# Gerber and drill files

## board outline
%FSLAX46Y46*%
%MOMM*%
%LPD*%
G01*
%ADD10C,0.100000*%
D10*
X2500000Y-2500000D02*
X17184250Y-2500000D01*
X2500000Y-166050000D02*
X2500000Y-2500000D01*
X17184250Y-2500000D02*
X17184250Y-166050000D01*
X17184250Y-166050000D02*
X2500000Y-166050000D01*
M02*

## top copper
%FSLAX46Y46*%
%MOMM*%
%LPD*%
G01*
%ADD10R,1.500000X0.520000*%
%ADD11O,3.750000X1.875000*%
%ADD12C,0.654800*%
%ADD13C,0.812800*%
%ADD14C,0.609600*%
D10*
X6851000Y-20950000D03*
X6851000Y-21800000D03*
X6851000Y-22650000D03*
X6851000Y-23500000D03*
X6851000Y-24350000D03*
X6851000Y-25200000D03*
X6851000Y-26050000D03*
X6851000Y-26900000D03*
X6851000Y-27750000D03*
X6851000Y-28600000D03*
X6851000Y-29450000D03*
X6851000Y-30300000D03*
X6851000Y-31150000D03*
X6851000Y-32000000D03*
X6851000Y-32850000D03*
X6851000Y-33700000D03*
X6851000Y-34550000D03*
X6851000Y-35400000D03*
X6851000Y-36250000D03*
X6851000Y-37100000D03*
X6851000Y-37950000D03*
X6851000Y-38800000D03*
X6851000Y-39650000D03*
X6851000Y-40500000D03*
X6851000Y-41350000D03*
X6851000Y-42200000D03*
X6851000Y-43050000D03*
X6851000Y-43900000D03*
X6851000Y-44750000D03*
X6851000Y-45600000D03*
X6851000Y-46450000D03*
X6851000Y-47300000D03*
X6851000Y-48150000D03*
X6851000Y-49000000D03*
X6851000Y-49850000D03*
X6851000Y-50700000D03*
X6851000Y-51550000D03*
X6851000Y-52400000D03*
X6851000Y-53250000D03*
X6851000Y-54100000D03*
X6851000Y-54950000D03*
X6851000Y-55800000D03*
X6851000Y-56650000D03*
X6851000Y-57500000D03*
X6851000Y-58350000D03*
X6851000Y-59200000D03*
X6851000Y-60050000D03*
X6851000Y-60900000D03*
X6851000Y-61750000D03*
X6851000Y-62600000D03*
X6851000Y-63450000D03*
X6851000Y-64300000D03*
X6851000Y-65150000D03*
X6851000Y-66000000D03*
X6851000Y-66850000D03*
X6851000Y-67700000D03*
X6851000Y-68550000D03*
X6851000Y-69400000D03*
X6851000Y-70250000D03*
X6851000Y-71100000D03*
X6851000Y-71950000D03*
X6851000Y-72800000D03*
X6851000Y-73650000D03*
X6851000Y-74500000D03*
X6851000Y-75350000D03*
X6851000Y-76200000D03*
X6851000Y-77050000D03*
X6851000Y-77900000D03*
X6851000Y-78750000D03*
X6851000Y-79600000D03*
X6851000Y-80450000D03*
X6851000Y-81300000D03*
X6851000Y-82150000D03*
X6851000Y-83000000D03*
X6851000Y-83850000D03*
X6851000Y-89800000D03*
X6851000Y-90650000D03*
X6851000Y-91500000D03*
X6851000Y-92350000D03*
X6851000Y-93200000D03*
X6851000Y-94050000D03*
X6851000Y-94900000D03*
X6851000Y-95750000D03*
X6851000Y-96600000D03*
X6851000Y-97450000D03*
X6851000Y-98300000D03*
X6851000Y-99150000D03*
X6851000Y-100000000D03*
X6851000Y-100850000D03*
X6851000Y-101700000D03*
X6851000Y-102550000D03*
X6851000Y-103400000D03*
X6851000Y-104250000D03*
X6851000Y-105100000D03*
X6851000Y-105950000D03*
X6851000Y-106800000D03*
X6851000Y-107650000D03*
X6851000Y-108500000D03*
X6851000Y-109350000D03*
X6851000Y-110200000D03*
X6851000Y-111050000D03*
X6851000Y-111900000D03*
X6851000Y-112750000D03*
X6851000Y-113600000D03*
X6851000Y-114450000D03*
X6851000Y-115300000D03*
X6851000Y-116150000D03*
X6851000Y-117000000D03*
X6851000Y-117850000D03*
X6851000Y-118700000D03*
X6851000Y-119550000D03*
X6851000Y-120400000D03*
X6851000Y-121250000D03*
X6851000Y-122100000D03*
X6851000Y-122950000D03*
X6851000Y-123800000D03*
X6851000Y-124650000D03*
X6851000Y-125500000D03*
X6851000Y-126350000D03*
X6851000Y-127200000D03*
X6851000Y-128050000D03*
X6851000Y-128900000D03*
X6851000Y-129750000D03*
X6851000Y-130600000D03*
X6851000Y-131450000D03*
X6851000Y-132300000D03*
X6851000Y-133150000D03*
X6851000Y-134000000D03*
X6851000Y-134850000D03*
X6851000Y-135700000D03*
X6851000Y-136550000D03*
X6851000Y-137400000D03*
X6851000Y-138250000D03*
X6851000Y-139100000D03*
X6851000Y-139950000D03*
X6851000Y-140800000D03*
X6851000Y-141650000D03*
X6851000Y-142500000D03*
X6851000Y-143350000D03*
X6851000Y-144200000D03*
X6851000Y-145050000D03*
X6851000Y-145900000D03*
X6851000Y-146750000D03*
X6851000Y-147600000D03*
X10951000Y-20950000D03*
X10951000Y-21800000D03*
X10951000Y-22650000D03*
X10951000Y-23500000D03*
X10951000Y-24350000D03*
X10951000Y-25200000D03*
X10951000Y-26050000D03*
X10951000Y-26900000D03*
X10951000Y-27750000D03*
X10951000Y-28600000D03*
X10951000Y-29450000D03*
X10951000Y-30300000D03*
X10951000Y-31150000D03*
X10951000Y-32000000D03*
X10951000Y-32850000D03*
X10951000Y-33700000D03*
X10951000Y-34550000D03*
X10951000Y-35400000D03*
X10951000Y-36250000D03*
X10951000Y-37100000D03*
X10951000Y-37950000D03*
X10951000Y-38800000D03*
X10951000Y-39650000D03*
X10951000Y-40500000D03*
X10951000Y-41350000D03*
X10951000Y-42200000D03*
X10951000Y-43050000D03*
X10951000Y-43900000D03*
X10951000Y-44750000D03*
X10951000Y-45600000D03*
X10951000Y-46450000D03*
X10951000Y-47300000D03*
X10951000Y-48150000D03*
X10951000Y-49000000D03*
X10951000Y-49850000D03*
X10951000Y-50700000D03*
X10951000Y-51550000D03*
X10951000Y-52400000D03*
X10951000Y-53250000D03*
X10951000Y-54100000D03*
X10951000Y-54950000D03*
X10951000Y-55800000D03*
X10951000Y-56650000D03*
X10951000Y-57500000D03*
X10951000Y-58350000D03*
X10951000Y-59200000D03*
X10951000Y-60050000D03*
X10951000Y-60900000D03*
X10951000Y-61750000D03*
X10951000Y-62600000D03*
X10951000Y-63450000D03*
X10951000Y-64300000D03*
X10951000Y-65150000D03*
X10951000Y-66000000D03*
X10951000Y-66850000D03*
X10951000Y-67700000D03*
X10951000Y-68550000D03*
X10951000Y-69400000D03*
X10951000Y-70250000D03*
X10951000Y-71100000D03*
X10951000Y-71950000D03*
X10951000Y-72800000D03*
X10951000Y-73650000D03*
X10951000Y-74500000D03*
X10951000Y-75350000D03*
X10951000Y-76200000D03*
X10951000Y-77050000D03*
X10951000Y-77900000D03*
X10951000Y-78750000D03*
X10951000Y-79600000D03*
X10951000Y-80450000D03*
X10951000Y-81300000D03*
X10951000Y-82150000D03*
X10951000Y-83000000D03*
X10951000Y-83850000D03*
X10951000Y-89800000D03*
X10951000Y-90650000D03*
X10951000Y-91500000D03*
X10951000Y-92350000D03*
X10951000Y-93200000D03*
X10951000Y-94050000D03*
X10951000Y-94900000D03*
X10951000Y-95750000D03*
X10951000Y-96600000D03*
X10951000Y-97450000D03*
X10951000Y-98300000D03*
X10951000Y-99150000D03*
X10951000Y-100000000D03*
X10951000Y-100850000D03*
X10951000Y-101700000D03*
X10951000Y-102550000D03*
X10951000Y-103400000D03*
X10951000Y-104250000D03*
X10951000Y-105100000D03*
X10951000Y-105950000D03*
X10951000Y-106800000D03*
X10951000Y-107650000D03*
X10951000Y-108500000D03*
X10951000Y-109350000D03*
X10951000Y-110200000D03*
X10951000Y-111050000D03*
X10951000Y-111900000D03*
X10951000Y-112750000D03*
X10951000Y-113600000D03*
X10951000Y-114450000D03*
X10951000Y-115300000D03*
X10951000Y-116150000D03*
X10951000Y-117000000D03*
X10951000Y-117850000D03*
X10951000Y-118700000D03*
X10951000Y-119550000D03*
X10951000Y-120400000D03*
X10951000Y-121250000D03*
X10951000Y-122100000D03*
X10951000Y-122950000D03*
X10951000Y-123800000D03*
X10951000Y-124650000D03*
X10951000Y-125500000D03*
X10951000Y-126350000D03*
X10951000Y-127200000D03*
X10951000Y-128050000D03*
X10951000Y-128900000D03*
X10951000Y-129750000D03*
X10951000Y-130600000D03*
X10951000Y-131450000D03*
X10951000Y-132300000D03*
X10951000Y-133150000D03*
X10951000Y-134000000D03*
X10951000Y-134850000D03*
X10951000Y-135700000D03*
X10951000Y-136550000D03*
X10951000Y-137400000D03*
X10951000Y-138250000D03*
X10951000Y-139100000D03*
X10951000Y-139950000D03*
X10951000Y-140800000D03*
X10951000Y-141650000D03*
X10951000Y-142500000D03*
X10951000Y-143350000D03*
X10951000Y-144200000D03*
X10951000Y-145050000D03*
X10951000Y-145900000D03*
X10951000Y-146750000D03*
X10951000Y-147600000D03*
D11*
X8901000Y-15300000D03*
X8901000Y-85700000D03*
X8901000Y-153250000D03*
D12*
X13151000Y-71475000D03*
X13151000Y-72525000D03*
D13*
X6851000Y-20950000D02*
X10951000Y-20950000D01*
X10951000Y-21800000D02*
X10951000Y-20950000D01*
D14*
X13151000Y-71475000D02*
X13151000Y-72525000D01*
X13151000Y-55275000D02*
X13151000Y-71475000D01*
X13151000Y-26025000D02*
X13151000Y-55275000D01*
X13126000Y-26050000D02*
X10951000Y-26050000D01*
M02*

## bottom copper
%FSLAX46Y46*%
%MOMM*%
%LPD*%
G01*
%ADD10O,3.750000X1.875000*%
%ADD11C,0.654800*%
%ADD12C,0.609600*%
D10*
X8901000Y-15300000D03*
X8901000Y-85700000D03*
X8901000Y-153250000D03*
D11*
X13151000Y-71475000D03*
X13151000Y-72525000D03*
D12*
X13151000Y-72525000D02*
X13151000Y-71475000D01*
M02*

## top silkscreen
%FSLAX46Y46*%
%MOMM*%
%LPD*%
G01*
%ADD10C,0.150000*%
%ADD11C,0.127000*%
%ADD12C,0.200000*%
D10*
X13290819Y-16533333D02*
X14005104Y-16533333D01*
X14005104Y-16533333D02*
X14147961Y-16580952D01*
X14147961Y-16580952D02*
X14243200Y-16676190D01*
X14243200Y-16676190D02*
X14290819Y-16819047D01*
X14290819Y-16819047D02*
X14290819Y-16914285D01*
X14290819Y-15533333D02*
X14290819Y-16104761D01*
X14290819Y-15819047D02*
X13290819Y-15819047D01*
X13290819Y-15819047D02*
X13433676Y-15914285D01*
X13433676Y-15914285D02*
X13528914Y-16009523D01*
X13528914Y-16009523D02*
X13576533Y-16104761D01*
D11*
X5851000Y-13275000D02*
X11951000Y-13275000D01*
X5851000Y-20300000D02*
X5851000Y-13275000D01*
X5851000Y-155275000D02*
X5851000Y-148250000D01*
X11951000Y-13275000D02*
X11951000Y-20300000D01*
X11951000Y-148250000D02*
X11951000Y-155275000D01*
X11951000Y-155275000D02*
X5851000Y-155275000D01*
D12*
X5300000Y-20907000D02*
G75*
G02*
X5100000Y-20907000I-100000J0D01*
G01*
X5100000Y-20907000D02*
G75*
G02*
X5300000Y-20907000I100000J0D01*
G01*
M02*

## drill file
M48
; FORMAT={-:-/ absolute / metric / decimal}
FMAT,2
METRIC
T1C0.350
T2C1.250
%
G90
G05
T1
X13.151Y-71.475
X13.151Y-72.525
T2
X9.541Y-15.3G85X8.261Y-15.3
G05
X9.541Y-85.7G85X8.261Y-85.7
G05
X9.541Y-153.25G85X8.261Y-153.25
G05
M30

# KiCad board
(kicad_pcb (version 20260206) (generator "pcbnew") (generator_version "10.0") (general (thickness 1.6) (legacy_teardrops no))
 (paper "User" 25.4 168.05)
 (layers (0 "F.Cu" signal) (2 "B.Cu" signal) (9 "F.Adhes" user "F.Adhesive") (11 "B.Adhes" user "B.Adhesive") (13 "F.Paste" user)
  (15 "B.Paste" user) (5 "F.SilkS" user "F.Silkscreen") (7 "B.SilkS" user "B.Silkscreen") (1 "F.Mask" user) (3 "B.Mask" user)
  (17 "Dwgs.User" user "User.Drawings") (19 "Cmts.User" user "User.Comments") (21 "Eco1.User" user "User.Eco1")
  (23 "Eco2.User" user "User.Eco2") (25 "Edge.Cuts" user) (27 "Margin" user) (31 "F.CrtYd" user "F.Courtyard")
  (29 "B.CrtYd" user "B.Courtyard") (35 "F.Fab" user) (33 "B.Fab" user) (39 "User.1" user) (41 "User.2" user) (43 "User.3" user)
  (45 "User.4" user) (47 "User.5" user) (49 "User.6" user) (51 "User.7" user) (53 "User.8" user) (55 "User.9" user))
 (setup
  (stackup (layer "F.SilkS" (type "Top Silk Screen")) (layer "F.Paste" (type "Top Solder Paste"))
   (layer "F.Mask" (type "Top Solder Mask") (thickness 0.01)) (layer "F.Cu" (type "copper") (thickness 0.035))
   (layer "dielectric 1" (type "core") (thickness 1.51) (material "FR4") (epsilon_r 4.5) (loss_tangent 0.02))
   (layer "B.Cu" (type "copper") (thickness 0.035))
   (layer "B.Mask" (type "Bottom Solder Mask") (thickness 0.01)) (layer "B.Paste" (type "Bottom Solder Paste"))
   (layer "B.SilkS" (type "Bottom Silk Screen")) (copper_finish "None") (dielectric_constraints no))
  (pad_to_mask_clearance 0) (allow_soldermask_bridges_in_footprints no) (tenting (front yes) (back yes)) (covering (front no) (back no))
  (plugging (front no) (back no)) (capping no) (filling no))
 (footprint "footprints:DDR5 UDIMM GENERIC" (layer "F.Cu") (at 8.901 84.275 -90)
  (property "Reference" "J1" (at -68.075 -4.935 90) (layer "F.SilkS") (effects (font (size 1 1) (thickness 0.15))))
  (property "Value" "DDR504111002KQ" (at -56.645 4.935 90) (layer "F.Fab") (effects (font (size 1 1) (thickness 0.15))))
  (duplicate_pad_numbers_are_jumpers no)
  (fp_line (start -71 3.05) (end -71 -3.05) (stroke (width 0.127) (type solid)) (layer "F.SilkS"))
  (fp_line (start -63.975 3.05) (end -71 3.05) (stroke (width 0.127) (type solid)) (layer "F.SilkS"))
  (fp_line (start 71 3.05) (end 63.975 3.05) (stroke (width 0.127) (type solid)) (layer "F.SilkS"))
  (fp_line (start -71 -3.05) (end -63.975 -3.05) (stroke (width 0.127) (type solid)) (layer "F.SilkS"))
  (fp_line (start 63.975 -3.05) (end 71 -3.05) (stroke (width 0.127) (type solid)) (layer "F.SilkS"))
  (fp_line (start 71 -3.05) (end 71 3.05) (stroke (width 0.127) (type solid)) (layer "F.SilkS"))
  (fp_circle (center -63.368 3.701) (end -63.268 3.701) (stroke (width 0.2) (type solid)) (fill no) (layer "F.SilkS"))
  (pad "01" smd rect (at -63.325 2.05 270) (size 0.52 1.5) (layers "F.Cu" "F.Mask" "F.Paste") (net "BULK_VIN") (solder_mask_margin 0.102))
  (pad "02" smd rect (at -62.475 2.05 270) (size 0.52 1.5) (layers "F.Cu" "F.Mask" "F.Paste") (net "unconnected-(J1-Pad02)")
   (solder_mask_margin 0.102))
  (pad "03" smd rect (at -61.625 2.05 270) (size 0.52 1.5) (layers "F.Cu" "F.Mask" "F.Paste") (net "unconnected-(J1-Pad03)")
   (solder_mask_margin 0.102))
  (pad "04" smd rect (at -60.775 2.05 270) (size 0.52 1.5) (layers "F.Cu" "F.Mask" "F.Paste") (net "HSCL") (solder_mask_margin 0.102))
  (pad "05" smd rect (at -59.925 2.05 270) (size 0.52 1.5) (layers "F.Cu" "F.Mask" "F.Paste") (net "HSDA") (solder_mask_margin 0.102))
  (pad "06" smd rect (at -59.075 2.05 270) (size 0.52 1.5) (layers "F.Cu" "F.Mask" "F.Paste") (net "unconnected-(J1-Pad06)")
   (solder_mask_margin 0.102))
  (pad "07" smd rect (at -58.225 2.05 270) (size 0.52 1.5) (layers "F.Cu" "F.Mask" "F.Paste") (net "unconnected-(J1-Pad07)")
   (solder_mask_margin 0.102))
  (pad "08" smd rect (at -57.375 2.05 270) (size 0.52 1.5) (layers "F.Cu" "F.Mask" "F.Paste") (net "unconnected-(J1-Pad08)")
   (solder_mask_margin 0.102))
  (pad "09" smd rect (at -56.525 2.05 270) (size 0.52 1.5) (layers "F.Cu" "F.Mask" "F.Paste") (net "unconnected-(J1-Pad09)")
   (solder_mask_margin 0.102))
  (pad "10" smd rect (at -55.675 2.05 270) (size 0.52 1.5) (layers "F.Cu" "F.Mask" "F.Paste") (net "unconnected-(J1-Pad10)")
   (solder_mask_margin 0.102))
  (pad "11" smd rect (at -54.825 2.05 270) (size 0.52 1.5) (layers "F.Cu" "F.Mask" "F.Paste") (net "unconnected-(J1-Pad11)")
   (solder_mask_margin 0.102))
  (pad "12" smd rect (at -53.975 2.05 270) (size 0.52 1.5) (layers "F.Cu" "F.Mask" "F.Paste") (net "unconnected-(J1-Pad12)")
   (solder_mask_margin 0.102))
  (pad "13" smd rect (at -53.125 2.05 270) (size 0.52 1.5) (layers "F.Cu" "F.Mask" "F.Paste") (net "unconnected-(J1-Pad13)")
   (solder_mask_margin 0.102))
  (pad "14" smd rect (at -52.275 2.05 270) (size 0.52 1.5) (layers "F.Cu" "F.Mask" "F.Paste") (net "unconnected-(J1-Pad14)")
   (solder_mask_margin 0.102))
  (pad "15" smd rect (at -51.425 2.05 270) (size 0.52 1.5) (layers "F.Cu" "F.Mask" "F.Paste") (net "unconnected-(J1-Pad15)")
   (solder_mask_margin 0.102))
  (pad "16" smd rect (at -50.575 2.05 270) (size 0.52 1.5) (layers "F.Cu" "F.Mask" "F.Paste") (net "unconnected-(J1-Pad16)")
   (solder_mask_margin 0.102))
  (pad "17" smd rect (at -49.725 2.05 270) (size 0.52 1.5) (layers "F.Cu" "F.Mask" "F.Paste") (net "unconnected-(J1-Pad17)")
   (solder_mask_margin 0.102))
  (pad "18" smd rect (at -48.875 2.05 270) (size 0.52 1.5) (layers "F.Cu" "F.Mask" "F.Paste") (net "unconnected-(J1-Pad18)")
   (solder_mask_margin 0.102))
  (pad "19" smd rect (at -48.025 2.05 270) (size 0.52 1.5) (layers "F.Cu" "F.Mask" "F.Paste") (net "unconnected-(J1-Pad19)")
   (solder_mask_margin 0.102))
  (pad "20" smd rect (at -47.175 2.05 270) (size 0.52 1.5) (layers "F.Cu" "F.Mask" "F.Paste") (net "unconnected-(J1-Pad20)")
   (solder_mask_margin 0.102))
  (pad "21" smd rect (at -46.325 2.05 270) (size 0.52 1.5) (layers "F.Cu" "F.Mask" "F.Paste") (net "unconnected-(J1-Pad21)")
   (solder_mask_margin 0.102))
  (pad "22" smd rect (at -45.475 2.05 270) (size 0.52 1.5) (layers "F.Cu" "F.Mask" "F.Paste") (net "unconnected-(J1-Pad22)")
   (solder_mask_margin 0.102))
  (pad "23" smd rect (at -44.625 2.05 270) (size 0.52 1.5) (layers "F.Cu" "F.Mask" "F.Paste") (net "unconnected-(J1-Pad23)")
   (solder_mask_margin 0.102))
  (pad "24" smd rect (at -43.775 2.05 270) (size 0.52 1.5) (layers "F.Cu" "F.Mask" "F.Paste") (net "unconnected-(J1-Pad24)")
   (solder_mask_margin 0.102))
  (pad "25" smd rect (at -42.925 2.05 270) (size 0.52 1.5) (layers "F.Cu" "F.Mask" "F.Paste") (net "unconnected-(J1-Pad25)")
   (solder_mask_margin 0.102))
  (pad "26" smd rect (at -42.075 2.05 270) (size 0.52 1.5) (layers "F.Cu" "F.Mask" "F.Paste") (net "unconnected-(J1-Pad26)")
   (solder_mask_margin 0.102))
  (pad "27" smd rect (at -41.225 2.05 270) (size 0.52 1.5) (layers "F.Cu" "F.Mask" "F.Paste") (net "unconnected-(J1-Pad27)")
   (solder_mask_margin 0.102))
  (pad "28" smd rect (at -40.375 2.05 270) (size 0.52 1.5) (layers "F.Cu" "F.Mask" "F.Paste") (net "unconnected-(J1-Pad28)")
   (solder_mask_margin 0.102))
  (pad "29" smd rect (at -39.525 2.05 270) (size 0.52 1.5) (layers "F.Cu" "F.Mask" "F.Paste") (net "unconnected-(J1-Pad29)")
   (solder_mask_margin 0.102))
  (pad "30" smd rect (at -38.675 2.05 270) (size 0.52 1.5) (layers "F.Cu" "F.Mask" "F.Paste") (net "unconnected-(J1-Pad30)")
   (solder_mask_margin 0.102))
  (pad "31" smd rect (at -37.825 2.05 270) (size 0.52 1.5) (layers "F.Cu" "F.Mask" "F.Paste") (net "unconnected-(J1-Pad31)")
   (solder_mask_margin 0.102))
  (pad "32" smd rect (at -36.975 2.05 270) (size 0.52 1.5) (layers "F.Cu" "F.Mask" "F.Paste") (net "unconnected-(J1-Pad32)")
   (solder_mask_margin 0.102))
  (pad "33" smd rect (at -36.125 2.05 270) (size 0.52 1.5) (layers "F.Cu" "F.Mask" "F.Paste") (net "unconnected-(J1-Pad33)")
   (solder_mask_margin 0.102))
  (pad "34" smd rect (at -35.275 2.05 270) (size 0.52 1.5) (layers "F.Cu" "F.Mask" "F.Paste") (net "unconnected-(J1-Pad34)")
   (solder_mask_margin 0.102))
  (pad "35" smd rect (at -34.425 2.05 270) (size 0.52 1.5) (layers "F.Cu" "F.Mask" "F.Paste") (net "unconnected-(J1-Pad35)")
   (solder_mask_margin 0.102))
  (pad "36" smd rect (at -33.575 2.05 270) (size 0.52 1.5) (layers "F.Cu" "F.Mask" "F.Paste") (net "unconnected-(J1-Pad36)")
   (solder_mask_margin 0.102))
  (pad "37" smd rect (at -32.725 2.05 270) (size 0.52 1.5) (layers "F.Cu" "F.Mask" "F.Paste") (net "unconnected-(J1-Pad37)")
   (solder_mask_margin 0.102))
  (pad "38" smd rect (at -31.875 2.05 270) (size 0.52 1.5) (layers "F.Cu" "F.Mask" "F.Paste") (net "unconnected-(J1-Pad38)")
   (solder_mask_margin 0.102))
  (pad "39" smd rect (at -31.025 2.05 270) (size 0.52 1.5) (layers "F.Cu" "F.Mask" "F.Paste") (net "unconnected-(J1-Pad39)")
   (solder_mask_margin 0.102))
  (pad "40" smd rect (at -30.175 2.05 270) (size 0.52 1.5) (layers "F.Cu" "F.Mask" "F.Paste") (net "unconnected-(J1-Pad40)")
   (solder_mask_margin 0.102))
  (pad "41" smd rect (at -29.325 2.05 270) (size 0.52 1.5) (layers "F.Cu" "F.Mask" "F.Paste") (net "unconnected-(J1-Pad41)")
   (solder_mask_margin 0.102))
  (pad "42" smd rect (at -28.475 2.05 270) (size 0.52 1.5) (layers "F.Cu" "F.Mask" "F.Paste") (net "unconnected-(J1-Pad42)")
   (solder_mask_margin 0.102))
  (pad "43" smd rect (at -27.625 2.05 270) (size 0.52 1.5) (layers "F.Cu" "F.Mask" "F.Paste") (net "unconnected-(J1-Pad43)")
   (solder_mask_margin 0.102))
  (pad "44" smd rect (at -26.775 2.05 270) (size 0.52 1.5) (layers "F.Cu" "F.Mask" "F.Paste") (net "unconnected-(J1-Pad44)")
   (solder_mask_margin 0.102))
  (pad "45" smd rect (at -25.925 2.05 270) (size 0.52 1.5) (layers "F.Cu" "F.Mask" "F.Paste") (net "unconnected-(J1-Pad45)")
   (solder_mask_margin 0.102))
  (pad "46" smd rect (at -25.075 2.05 270) (size 0.52 1.5) (layers "F.Cu" "F.Mask" "F.Paste") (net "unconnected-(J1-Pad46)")
   (solder_mask_margin 0.102))
  (pad "47" smd rect (at -24.225 2.05 270) (size 0.52 1.5) (layers "F.Cu" "F.Mask" "F.Paste") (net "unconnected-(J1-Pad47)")
   (solder_mask_margin 0.102))
  (pad "48" smd rect (at -23.375 2.05 270) (size 0.52 1.5) (layers "F.Cu" "F.Mask" "F.Paste") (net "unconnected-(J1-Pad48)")
   (solder_mask_margin 0.102))
  (pad "49" smd rect (at -22.525 2.05 270) (size 0.52 1.5) (layers "F.Cu" "F.Mask" "F.Paste") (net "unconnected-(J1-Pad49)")
   (solder_mask_margin 0.102))
  (pad "50" smd rect (at -21.675 2.05 270) (size 0.52 1.5) (layers "F.Cu" "F.Mask" "F.Paste") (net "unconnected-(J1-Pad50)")
   (solder_mask_margin 0.102))
  (pad "51" smd rect (at -20.825 2.05 270) (size 0.52 1.5) (layers "F.Cu" "F.Mask" "F.Paste") (solder_mask_margin 0.102))
  (pad "52" smd rect (at -19.975 2.05 270) (size 0.52 1.5) (layers "F.Cu" "F.Mask" "F.Paste") (solder_mask_margin 0.102))
  (pad "53" smd rect (at -19.125 2.05 270) (size 0.52 1.5) (layers "F.Cu" "F.Mask" "F.Paste") (solder_mask_margin 0.102))
  (pad "54" smd rect (at -18.275 2.05 270) (size 0.52 1.5) (layers "F.Cu" "F.Mask" "F.Paste") (solder_mask_margin 0.102))
  (pad "55" smd rect (at -17.425 2.05 270) (size 0.52 1.5) (layers "F.Cu" "F.Mask" "F.Paste") (solder_mask_margin 0.102))
  (pad "56" smd rect (at -16.575 2.05 270) (size 0.52 1.5) (layers "F.Cu" "F.Mask" "F.Paste") (solder_mask_margin 0.102))
  (pad "57" smd rect (at -15.725 2.05 270) (size 0.52 1.5) (layers "F.Cu" "F.Mask" "F.Paste") (solder_mask_margin 0.102))
  (pad "58" smd rect (at -14.875 2.05 270) (size 0.52 1.5) (layers "F.Cu" "F.Mask" "F.Paste") (solder_mask_margin 0.102))
  (pad "59" smd rect (at -14.025 2.05 270) (size 0.52 1.5) (layers "F.Cu" "F.Mask" "F.Paste") (solder_mask_margin 0.102))
  (pad "60" smd rect (at -13.175 2.05 270) (size 0.52 1.5) (layers "F.Cu" "F.Mask" "F.Paste") (solder_mask_margin 0.102))
  (pad "61" smd rect (at -12.325 2.05 270) (size 0.52 1.5) (layers "F.Cu" "F.Mask" "F.Paste") (solder_mask_margin 0.102))
  (pad "62" smd rect (at -11.475 2.05 270) (size 0.52 1.5) (layers "F.Cu" "F.Mask" "F.Paste") (solder_mask_margin 0.102))
  (pad "63" smd rect (at -10.625 2.05 270) (size 0.52 1.5) (layers "F.Cu" "F.Mask" "F.Paste") (solder_mask_margin 0.102))
  (pad "64" smd rect (at -9.775 2.05 270) (size 0.52 1.5) (layers "F.Cu" "F.Mask" "F.Paste") (solder_mask_margin 0.102))
  (pad "65" smd rect (at -8.925 2.05 270) (size 0.52 1.5) (layers "F.Cu" "F.Mask" "F.Paste") (solder_mask_margin 0.102))
  (pad "66" smd rect (at -8.075 2.05 270) (size 0.52 1.5) (layers "F.Cu" "F.Mask" "F.Paste") (solder_mask_margin 0.102))
  (pad "67" smd rect (at -7.225 2.05 270) (size 0.52 1.5) (layers "F.Cu" "F.Mask" "F.Paste") (solder_mask_margin 0.102))
  (pad "68" smd rect (at -6.375 2.05 270) (size 0.52 1.5) (layers "F.Cu" "F.Mask" "F.Paste") (solder_mask_margin 0.102))
  (pad "69" smd rect (at -5.525 2.05 270) (size 0.52 1.5) (layers "F.Cu" "F.Mask" "F.Paste") (solder_mask_margin 0.102))
  (pad "70" smd rect (at -4.675 2.05 270) (size 0.52 1.5) (layers "F.Cu" "F.Mask" "F.Paste") (solder_mask_margin 0.102))
  (pad "71" smd rect (at -3.825 2.05 270) (size 0.52 1.5) (layers "F.Cu" "F.Mask" "F.Paste") (solder_mask_margin 0.102))
  (pad "72" smd rect (at -2.975 2.05 270) (size 0.52 1.5) (layers "F.Cu" "F.Mask" "F.Paste") (solder_mask_margin 0.102))
  (pad "73" smd rect (at -2.125 2.05 270) (size 0.52 1.5) (layers "F.Cu" "F.Mask" "F.Paste") (solder_mask_margin 0.102))
  (pad "74" smd rect (at -1.275 2.05 270) (size 0.52 1.5) (layers "F.Cu" "F.Mask" "F.Paste") (solder_mask_margin 0.102))
  (pad "75" smd rect (at -0.425 2.05 270) (size 0.52 1.5) (layers "F.Cu" "F.Mask" "F.Paste") (solder_mask_margin 0.102))
  (pad "76" smd rect (at 5.525 2.05 270) (size 0.52 1.5) (layers "F.Cu" "F.Mask" "F.Paste") (solder_mask_margin 0.102))
  (pad "77" smd rect (at 6.375 2.05 270) (size 0.52 1.5) (layers "F.Cu" "F.Mask" "F.Paste") (solder_mask_margin 0.102))
  (pad "78" smd rect (at 7.225 2.05 270) (size 0.52 1.5) (layers "F.Cu" "F.Mask" "F.Paste") (solder_mask_margin 0.102))
  (pad "79" smd rect (at 8.075 2.05 270) (size 0.52 1.5) (layers "F.Cu" "F.Mask" "F.Paste") (solder_mask_margin 0.102))
  (pad "80" smd rect (at 8.925 2.05 270) (size 0.52 1.5) (layers "F.Cu" "F.Mask" "F.Paste") (solder_mask_margin 0.102))
  (pad "81" smd rect (at 9.775 2.05 270) (size 0.52 1.5) (layers "F.Cu" "F.Mask" "F.Paste") (solder_mask_margin 0.102))
  (pad "82" smd rect (at 10.625 2.05 270) (size 0.52 1.5) (layers "F.Cu" "F.Mask" "F.Paste") (solder_mask_margin 0.102))
  (pad "83" smd rect (at 11.475 2.05 270) (size 0.52 1.5) (layers "F.Cu" "F.Mask" "F.Paste") (solder_mask_margin 0.102))
  (pad "84" smd rect (at 12.325 2.05 270) (size 0.52 1.5) (layers "F.Cu" "F.Mask" "F.Paste") (solder_mask_margin 0.102))
  (pad "85" smd rect (at 13.175 2.05 270) (size 0.52 1.5) (layers "F.Cu" "F.Mask" "F.Paste") (solder_mask_margin 0.102))
  (pad "86" smd rect (at 14.025 2.05 270) (size 0.52 1.5) (layers "F.Cu" "F.Mask" "F.Paste") (solder_mask_margin 0.102))
  (pad "87" smd rect (at 14.875 2.05 270) (size 0.52 1.5) (layers "F.Cu" "F.Mask" "F.Paste") (solder_mask_margin 0.102))
  (pad "88" smd rect (at 15.725 2.05 270) (size 0.52 1.5) (layers "F.Cu" "F.Mask" "F.Paste") (solder_mask_margin 0.102))
  (pad "89" smd rect (at 16.575 2.05 270) (size 0.52 1.5) (layers "F.Cu" "F.Mask" "F.Paste") (solder_mask_margin 0.102))
  (pad "90" smd rect (at 17.425 2.05 270) (size 0.52 1.5) (layers "F.Cu" "F.Mask" "F.Paste") (solder_mask_margin 0.102))
  (pad "91" smd rect (at 18.275 2.05 270) (size 0.52 1.5) (layers "F.Cu" "F.Mask" "F.Paste") (solder_mask_margin 0.102))
  (pad "92" smd rect (at 19.125 2.05 270) (size 0.52 1.5) (layers "F.Cu" "F.Mask" "F.Paste") (solder_mask_margin 0.102))
  (pad "93" smd rect (at 19.975 2.05 270) (size 0.52 1.5) (layers "F.Cu" "F.Mask" "F.Paste") (solder_mask_margin 0.102))
  (pad "94" smd rect (at 20.825 2.05 270) (size 0.52 1.5) (layers "F.Cu" "F.Mask" "F.Paste") (solder_mask_margin 0.102))
  (pad "95" smd rect (at 21.675 2.05 270) (size 0.52 1.5) (layers "F.Cu" "F.Mask" "F.Paste") (solder_mask_margin 0.102))
  (pad "96" smd rect (at 22.525 2.05 270) (size 0.52 1.5) (layers "F.Cu" "F.Mask" "F.Paste") (solder_mask_margin 0.102))
  (pad "97" smd rect (at 23.375 2.05 270) (size 0.52 1.5) (layers "F.Cu" "F.Mask" "F.Paste") (solder_mask_margin 0.102))
  (pad "98" smd rect (at 24.225 2.05 270) (size 0.52 1.5) (layers "F.Cu" "F.Mask" "F.Paste") (solder_mask_margin 0.102))
  (pad "99" smd rect (at 25.075 2.05 270) (size 0.52 1.5) (layers "F.Cu" "F.Mask" "F.Paste") (solder_mask_margin 0.102))
  (pad "100" smd rect (at 25.925 2.05 270) (size 0.52 1.5) (layers "F.Cu" "F.Mask" "F.Paste") (solder_mask_margin 0.102))
  (pad "101" smd rect (at 26.775 2.05 270) (size 0.52 1.5) (layers "F.Cu" "F.Mask" "F.Paste") (solder_mask_margin 0.102))
  (pad "102" smd rect (at 27.625 2.05 270) (size 0.52 1.5) (layers "F.Cu" "F.Mask" "F.Paste") (solder_mask_margin 0.102))
  (pad "103" smd rect (at 28.475 2.05 270) (size 0.52 1.5) (layers "F.Cu" "F.Mask" "F.Paste") (solder_mask_margin 0.102))
  (pad "104" smd rect (at 29.325 2.05 270) (size 0.52 1.5) (layers "F.Cu" "F.Mask" "F.Paste") (solder_mask_margin 0.102))
  (pad "105" smd rect (at 30.175 2.05 270) (size 0.52 1.5) (layers "F.Cu" "F.Mask" "F.Paste") (solder_mask_margin 0.102))
  (pad "106" smd rect (at 31.025 2.05 270) (size 0.52 1.5) (layers "F.Cu" "F.Mask" "F.Paste") (solder_mask_margin 0.102))
  (pad "107" smd rect (at 31.875 2.05 270) (size 0.52 1.5) (layers "F.Cu" "F.Mask" "F.Paste") (solder_mask_margin 0.102))
  (pad "108" smd rect (at 32.725 2.05 270) (size 0.52 1.5) (layers "F.Cu" "F.Mask" "F.Paste") (solder_mask_margin 0.102))
  (pad "109" smd rect (at 33.575 2.05 270) (size 0.52 1.5) (layers "F.Cu" "F.Mask" "F.Paste") (solder_mask_margin 0.102))
  (pad "110" smd rect (at 34.425 2.05 270) (size 0.52 1.5) (layers "F.Cu" "F.Mask" "F.Paste") (solder_mask_margin 0.102))
  (pad "111" smd rect (at 35.275 2.05 270) (size 0.52 1.5) (layers "F.Cu" "F.Mask" "F.Paste") (solder_mask_margin 0.102))
  (pad "112" smd rect (at 36.125 2.05 270) (size 0.52 1.5) (layers "F.Cu" "F.Mask" "F.Paste") (solder_mask_margin 0.102))
  (pad "113" smd rect (at 36.975 2.05 270) (size 0.52 1.5) (layers "F.Cu" "F.Mask" "F.Paste") (solder_mask_margin 0.102))
  (pad "114" smd rect (at 37.825 2.05 270) (size 0.52 1.5) (layers "F.Cu" "F.Mask" "F.Paste") (solder_mask_margin 0.102))
  (pad "115" smd rect (at 38.675 2.05 270) (size 0.52 1.5) (layers "F.Cu" "F.Mask" "F.Paste") (solder_mask_margin 0.102))
  (pad "116" smd rect (at 39.525 2.05 270) (size 0.52 1.5) (layers "F.Cu" "F.Mask" "F.Paste") (solder_mask_margin 0.102))
  (pad "117" smd rect (at 40.375 2.05 270) (size 0.52 1.5) (layers "F.Cu" "F.Mask" "F.Paste") (solder_mask_margin 0.102))
  (pad "118" smd rect (at 41.225 2.05 270) (size 0.52 1.5) (layers "F.Cu" "F.Mask" "F.Paste") (solder_mask_margin 0.102))
  (pad "119" smd rect (at 42.075 2.05 270) (size 0.52 1.5) (layers "F.Cu" "F.Mask" "F.Paste") (solder_mask_margin 0.102))
  (pad "120" smd rect (at 42.925 2.05 270) (size 0.52 1.5) (layers "F.Cu" "F.Mask" "F.Paste") (solder_mask_margin 0.102))
  (pad "121" smd rect (at 43.775 2.05 270) (size 0.52 1.5) (layers "F.Cu" "F.Mask" "F.Paste") (solder_mask_margin 0.102))
  (pad "122" smd rect (at 44.625 2.05 270) (size 0.52 1.5) (layers "F.Cu" "F.Mask" "F.Paste") (solder_mask_margin 0.102))
  (pad "123" smd rect (at 45.475 2.05 270) (size 0.52 1.5) (layers "F.Cu" "F.Mask" "F.Paste") (solder_mask_margin 0.102))
  (pad "124" smd rect (at 46.325 2.05 270) (size 0.52 1.5) (layers "F.Cu" "F.Mask" "F.Paste") (solder_mask_margin 0.102))
  (pad "125" smd rect (at 47.175 2.05 270) (size 0.52 1.5) (layers "F.Cu" "F.Mask" "F.Paste") (solder_mask_margin 0.102))
  (pad "126" smd rect (at 48.025 2.05 270) (size 0.52 1.5) (layers "F.Cu" "F.Mask" "F.Paste") (solder_mask_margin 0.102))
  (pad "127" smd rect (at 48.875 2.05 270) (size 0.52 1.5) (layers "F.Cu" "F.Mask" "F.Paste") (solder_mask_margin 0.102))
  (pad "128" smd rect (at 49.725 2.05 270) (size 0.52 1.5) (layers "F.Cu" "F.Mask" "F.Paste") (solder_mask_margin 0.102))
  (pad "129" smd rect (at 50.575 2.05 270) (size 0.52 1.5) (layers "F.Cu" "F.Mask" "F.Paste") (solder_mask_margin 0.102))
  (pad "130" smd rect (at 51.425 2.05 270) (size 0.52 1.5) (layers "F.Cu" "F.Mask" "F.Paste") (solder_mask_margin 0.102))
  (pad "131" smd rect (at 52.275 2.05 270) (size 0.52 1.5) (layers "F.Cu" "F.Mask" "F.Paste") (solder_mask_margin 0.102))
  (pad "132" smd rect (at 53.125 2.05 270) (size 0.52 1.5) (layers "F.Cu" "F.Mask" "F.Paste") (solder_mask_margin 0.102))
  (pad "133" smd rect (at 53.975 2.05 270) (size 0.52 1.5) (layers "F.Cu" "F.Mask" "F.Paste") (solder_mask_margin 0.102))
  (pad "134" smd rect (at 54.825 2.05 270) (size 0.52 1.5) (layers "F.Cu" "F.Mask" "F.Paste") (solder_mask_margin 0.102))
  (pad "135" smd rect (at 55.675 2.05 270) (size 0.52 1.5) (layers "F.Cu" "F.Mask" "F.Paste") (solder_mask_margin 0.102))
  (pad "136" smd rect (at 56.525 2.05 270) (size 0.52 1.5) (layers "F.Cu" "F.Mask" "F.Paste") (solder_mask_margin 0.102))
  (pad "137" smd rect (at 57.375 2.05 270) (size 0.52 1.5) (layers "F.Cu" "F.Mask" "F.Paste") (solder_mask_margin 0.102))
  (pad "138" smd rect (at 58.225 2.05 270) (size 0.52 1.5) (layers "F.Cu" "F.Mask" "F.Paste") (solder_mask_margin 0.102))
  (pad "139" smd rect (at 59.075 2.05 270) (size 0.52 1.5) (layers "F.Cu" "F.Mask" "F.Paste") (solder_mask_margin 0.102))
  (pad "140" smd rect (at 59.925 2.05 270) (size 0.52 1.5) (layers "F.Cu" "F.Mask" "F.Paste") (solder_mask_margin 0.102))
  (pad "141" smd rect (at 60.775 2.05 270) (size 0.52 1.5) (layers "F.Cu" "F.Mask" "F.Paste") (solder_mask_margin 0.102))
  (pad "142" smd rect (at 61.625 2.05 270) (size 0.52 1.5) (layers "F.Cu" "F.Mask" "F.Paste") (solder_mask_margin 0.102))
  (pad "143" smd rect (at 62.475 2.05 270) (size 0.52 1.5) (layers "F.Cu" "F.Mask" "F.Paste") (solder_mask_margin 0.102))
  (pad "144" smd rect (at 63.325 2.05 270) (size 0.52 1.5) (layers "F.Cu" "F.Mask" "F.Paste") (solder_mask_margin 0.102))
  (pad "145" smd rect (at -63.325 -2.05 270) (size 0.52 1.5) (layers "F.Cu" "F.Mask" "F.Paste") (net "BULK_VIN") (solder_mask_margin 0.102))
  (pad "146" smd rect (at -62.475 -2.05 270) (size 0.52 1.5) (layers "F.Cu" "F.Mask" "F.Paste") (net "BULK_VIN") (solder_mask_margin 0.102))
  (pad "147" smd rect (at -61.625 -2.05 270) (size 0.52 1.5) (layers "F.Cu" "F.Mask" "F.Paste") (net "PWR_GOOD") (solder_mask_margin 0.102))
  (pad "148" smd rect (at -60.775 -2.05 270) (size 0.52 1.5) (layers "F.Cu" "F.Mask" "F.Paste") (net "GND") (solder_mask_margin 0.102))
  (pad "149" smd rect (at -59.925 -2.05 270) (size 0.52 1.5) (layers "F.Cu" "F.Mask" "F.Paste") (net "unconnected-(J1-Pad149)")
   (solder_mask_margin 0.102))
  (pad "150" smd rect (at -59.075 -2.05 270) (size 0.52 1.5) (layers "F.Cu" "F.Mask" "F.Paste") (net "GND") (solder_mask_margin 0.102))
  (pad "151" smd rect (at -58.225 -2.05 270) (size 0.52 1.5) (layers "F.Cu" "F.Mask" "F.Paste") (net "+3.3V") (solder_mask_margin 0.102))
  (pad "152" smd rect (at -57.375 -2.05 270) (size 0.52 1.5) (layers "F.Cu" "F.Mask" "F.Paste") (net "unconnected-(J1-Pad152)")
   (solder_mask_margin 0.102))
  (pad "153" smd rect (at -56.525 -2.05 270) (size 0.52 1.5) (layers "F.Cu" "F.Mask" "F.Paste") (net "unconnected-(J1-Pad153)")
   (solder_mask_margin 0.102))
  (pad "154" smd rect (at -55.675 -2.05 270) (size 0.52 1.5) (layers "F.Cu" "F.Mask" "F.Paste") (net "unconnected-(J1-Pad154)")
   (solder_mask_margin 0.102))
  (pad "155" smd rect (at -54.825 -2.05 270) (size 0.52 1.5) (layers "F.Cu" "F.Mask" "F.Paste") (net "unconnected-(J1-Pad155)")
   (solder_mask_margin 0.102))
  (pad "156" smd rect (at -53.975 -2.05 270) (size 0.52 1.5) (layers "F.Cu" "F.Mask" "F.Paste") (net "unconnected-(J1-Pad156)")
   (solder_mask_margin 0.102))
  (pad "157" smd rect (at -53.125 -2.05 270) (size 0.52 1.5) (layers "F.Cu" "F.Mask" "F.Paste") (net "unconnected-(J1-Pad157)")
   (solder_mask_margin 0.102))
  (pad "158" smd rect (at -52.275 -2.05 270) (size 0.52 1.5) (layers "F.Cu" "F.Mask" "F.Paste") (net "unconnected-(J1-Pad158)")
   (solder_mask_margin 0.102))
  (pad "159" smd rect (at -51.425 -2.05 270) (size 0.52 1.5) (layers "F.Cu" "F.Mask" "F.Paste") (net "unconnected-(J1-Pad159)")
   (solder_mask_margin 0.102))
  (pad "160" smd rect (at -50.575 -2.05 270) (size 0.52 1.5) (layers "F.Cu" "F.Mask" "F.Paste") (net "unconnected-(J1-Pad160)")
   (solder_mask_margin 0.102))
  (pad "161" smd rect (at -49.725 -2.05 270) (size 0.52 1.5) (layers "F.Cu" "F.Mask" "F.Paste") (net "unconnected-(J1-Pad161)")
   (solder_mask_margin 0.102))
  (pad "162" smd rect (at -48.875 -2.05 270) (size 0.52 1.5) (layers "F.Cu" "F.Mask" "F.Paste") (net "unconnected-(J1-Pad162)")
   (solder_mask_margin 0.102))
  (pad "163" smd rect (at -48.025 -2.05 270) (size 0.52 1.5) (layers "F.Cu" "F.Mask" "F.Paste") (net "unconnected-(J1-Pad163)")
   (solder_mask_margin 0.102))
  (pad "164" smd rect (at -47.175 -2.05 270) (size 0.52 1.5) (layers "F.Cu" "F.Mask" "F.Paste") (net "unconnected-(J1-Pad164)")
   (solder_mask_margin 0.102))
  (pad "165" smd rect (at -46.325 -2.05 270) (size 0.52 1.5) (layers "F.Cu" "F.Mask" "F.Paste") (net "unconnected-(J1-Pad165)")
   (solder_mask_margin 0.102))
  (pad "166" smd rect (at -45.475 -2.05 270) (size 0.52 1.5) (layers "F.Cu" "F.Mask" "F.Paste") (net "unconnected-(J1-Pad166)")
   (solder_mask_margin 0.102))
  (pad "167" smd rect (at -44.625 -2.05 270) (size 0.52 1.5) (layers "F.Cu" "F.Mask" "F.Paste") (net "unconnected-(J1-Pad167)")
   (solder_mask_margin 0.102))
  (pad "168" smd rect (at -43.775 -2.05 270) (size 0.52 1.5) (layers "F.Cu" "F.Mask" "F.Paste") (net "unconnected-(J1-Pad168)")
   (solder_mask_margin 0.102))
  (pad "169" smd rect (at -42.925 -2.05 270) (size 0.52 1.5) (layers "F.Cu" "F.Mask" "F.Paste") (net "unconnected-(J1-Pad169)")
   (solder_mask_margin 0.102))
  (pad "170" smd rect (at -42.075 -2.05 270) (size 0.52 1.5) (layers "F.Cu" "F.Mask" "F.Paste") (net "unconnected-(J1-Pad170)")
   (solder_mask_margin 0.102))
  (pad "171" smd rect (at -41.225 -2.05 270) (size 0.52 1.5) (layers "F.Cu" "F.Mask" "F.Paste") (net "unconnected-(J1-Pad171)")
   (solder_mask_margin 0.102))
  (pad "172" smd rect (at -40.375 -2.05 270) (size 0.52 1.5) (layers "F.Cu" "F.Mask" "F.Paste") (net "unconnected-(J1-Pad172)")
   (solder_mask_margin 0.102))
  (pad "173" smd rect (at -39.525 -2.05 270) (size 0.52 1.5) (layers "F.Cu" "F.Mask" "F.Paste") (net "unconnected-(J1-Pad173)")
   (solder_mask_margin 0.102))
  (pad "174" smd rect (at -38.675 -2.05 270) (size 0.52 1.5) (layers "F.Cu" "F.Mask" "F.Paste") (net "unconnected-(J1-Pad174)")
   (solder_mask_margin 0.102))
  (pad "175" smd rect (at -37.825 -2.05 270) (size 0.52 1.5) (layers "F.Cu" "F.Mask" "F.Paste") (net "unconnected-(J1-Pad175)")
   (solder_mask_margin 0.102))
  (pad "176" smd rect (at -36.975 -2.05 270) (size 0.52 1.5) (layers "F.Cu" "F.Mask" "F.Paste") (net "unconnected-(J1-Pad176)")
   (solder_mask_margin 0.102))
  (pad "177" smd rect (at -36.125 -2.05 270) (size 0.52 1.5) (layers "F.Cu" "F.Mask" "F.Paste") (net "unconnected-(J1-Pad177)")
   (solder_mask_margin 0.102))
  (pad "178" smd rect (at -35.275 -2.05 270) (size 0.52 1.5) (layers "F.Cu" "F.Mask" "F.Paste") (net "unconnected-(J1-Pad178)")
   (solder_mask_margin 0.102))
  (pad "179" smd rect (at -34.425 -2.05 270) (size 0.52 1.5) (layers "F.Cu" "F.Mask" "F.Paste") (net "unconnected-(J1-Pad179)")
   (solder_mask_margin 0.102))
  (pad "180" smd rect (at -33.575 -2.05 270) (size 0.52 1.5) (layers "F.Cu" "F.Mask" "F.Paste") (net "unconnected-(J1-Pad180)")
   (solder_mask_margin 0.102))
  (pad "181" smd rect (at -32.725 -2.05 270) (size 0.52 1.5) (layers "F.Cu" "F.Mask" "F.Paste") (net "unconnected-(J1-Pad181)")
   (solder_mask_margin 0.102))
  (pad "182" smd rect (at -31.875 -2.05 270) (size 0.52 1.5) (layers "F.Cu" "F.Mask" "F.Paste") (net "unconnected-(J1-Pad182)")
   (solder_mask_margin 0.102))
  (pad "183" smd rect (at -31.025 -2.05 270) (size 0.52 1.5) (layers "F.Cu" "F.Mask" "F.Paste") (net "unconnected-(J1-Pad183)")
   (solder_mask_margin 0.102))
  (pad "184" smd rect (at -30.175 -2.05 270) (size 0.52 1.5) (layers "F.Cu" "F.Mask" "F.Paste") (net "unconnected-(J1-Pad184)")
   (solder_mask_margin 0.102))
  (pad "185" smd rect (at -29.325 -2.05 270) (size 0.52 1.5) (layers "F.Cu" "F.Mask" "F.Paste") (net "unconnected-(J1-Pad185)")
   (solder_mask_margin 0.102))
  (pad "186" smd rect (at -28.475 -2.05 270) (size 0.52 1.5) (layers "F.Cu" "F.Mask" "F.Paste") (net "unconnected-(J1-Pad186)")
   (solder_mask_margin 0.102))
  (pad "187" smd rect (at -27.625 -2.05 270) (size 0.52 1.5) (layers "F.Cu" "F.Mask" "F.Paste") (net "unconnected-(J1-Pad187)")
   (solder_mask_margin 0.102))
  (pad "188" smd rect (at -26.775 -2.05 270) (size 0.52 1.5) (layers "F.Cu" "F.Mask" "F.Paste") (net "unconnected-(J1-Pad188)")
   (solder_mask_margin 0.102))
  (pad "189" smd rect (at -25.925 -2.05 270) (size 0.52 1.5) (layers "F.Cu" "F.Mask" "F.Paste") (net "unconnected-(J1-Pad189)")
   (solder_mask_margin 0.102))
  (pad "190" smd rect (at -25.075 -2.05 270) (size 0.52 1.5) (layers "F.Cu" "F.Mask" "F.Paste") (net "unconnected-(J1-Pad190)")
   (solder_mask_margin 0.102))
  (pad "191" smd rect (at -24.225 -2.05 270) (size 0.52 1.5) (layers "F.Cu" "F.Mask" "F.Paste") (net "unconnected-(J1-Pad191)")
   (solder_mask_margin 0.102))
  (pad "192" smd rect (at -23.375 -2.05 270) (size 0.52 1.5) (layers "F.Cu" "F.Mask" "F.Paste") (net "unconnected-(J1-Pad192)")
   (solder_mask_margin 0.102))
  (pad "193" smd rect (at -22.525 -2.05 270) (size 0.52 1.5) (layers "F.Cu" "F.Mask" "F.Paste") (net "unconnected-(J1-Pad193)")
   (solder_mask_margin 0.102))
  (pad "194" smd rect (at -21.675 -2.05 270) (size 0.52 1.5) (layers "F.Cu" "F.Mask" "F.Paste") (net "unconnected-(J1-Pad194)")
   (solder_mask_margin 0.102))
  (pad "195" smd rect (at -20.825 -2.05 270) (size 0.52 1.5) (layers "F.Cu" "F.Mask" "F.Paste") (solder_mask_margin 0.102))
  (pad "196" smd rect (at -19.975 -2.05 270) (size 0.52 1.5) (layers "F.Cu" "F.Mask" "F.Paste") (solder_mask_margin 0.102))
  (pad "197" smd rect (at -19.125 -2.05 270) (size 0.52 1.5) (layers "F.Cu" "F.Mask" "F.Paste") (solder_mask_margin 0.102))
  (pad "198" smd rect (at -18.275 -2.05 270) (size 0.52 1.5) (layers "F.Cu" "F.Mask" "F.Paste") (solder_mask_margin 0.102))
  (pad "199" smd rect (at -17.425 -2.05 270) (size 0.52 1.5) (layers "F.Cu" "F.Mask" "F.Paste") (solder_mask_margin 0.102))
  (pad "200" smd rect (at -16.575 -2.05 270) (size 0.52 1.5) (layers "F.Cu" "F.Mask" "F.Paste") (solder_mask_margin 0.102))
  (pad "201" smd rect (at -15.725 -2.05 270) (size 0.52 1.5) (layers "F.Cu" "F.Mask" "F.Paste") (solder_mask_margin 0.102))
  (pad "202" smd rect (at -14.875 -2.05 270) (size 0.52 1.5) (layers "F.Cu" "F.Mask" "F.Paste") (solder_mask_margin 0.102))
  (pad "203" smd rect (at -14.025 -2.05 270) (size 0.52 1.5) (layers "F.Cu" "F.Mask" "F.Paste") (solder_mask_margin 0.102))
  (pad "204" smd rect (at -13.175 -2.05 270) (size 0.52 1.5) (layers "F.Cu" "F.Mask" "F.Paste") (solder_mask_margin 0.102))
  (pad "205" smd rect (at -12.325 -2.05 270) (size 0.52 1.5) (layers "F.Cu" "F.Mask" "F.Paste") (solder_mask_margin 0.102))
  (pad "206" smd rect (at -11.475 -2.05 270) (size 0.52 1.5) (layers "F.Cu" "F.Mask" "F.Paste") (solder_mask_margin 0.102))
  (pad "207" smd rect (at -10.625 -2.05 270) (size 0.52 1.5) (layers "F.Cu" "F.Mask" "F.Paste") (solder_mask_margin 0.102))
  (pad "208" smd rect (at -9.775 -2.05 270) (size 0.52 1.5) (layers "F.Cu" "F.Mask" "F.Paste") (solder_mask_margin 0.102))
  (pad "209" smd rect (at -8.925 -2.05 270) (size 0.52 1.5) (layers "F.Cu" "F.Mask" "F.Paste") (solder_mask_margin 0.102))
  (pad "210" smd rect (at -8.075 -2.05 270) (size 0.52 1.5) (layers "F.Cu" "F.Mask" "F.Paste") (solder_mask_margin 0.102))
  (pad "211" smd rect (at -7.225 -2.05 270) (size 0.52 1.5) (layers "F.Cu" "F.Mask" "F.Paste") (solder_mask_margin 0.102))
  (pad "212" smd rect (at -6.375 -2.05 270) (size 0.52 1.5) (layers "F.Cu" "F.Mask" "F.Paste") (solder_mask_margin 0.102))
  (pad "213" smd rect (at -5.525 -2.05 270) (size 0.52 1.5) (layers "F.Cu" "F.Mask" "F.Paste") (solder_mask_margin 0.102))
  (pad "214" smd rect (at -4.675 -2.05 270) (size 0.52 1.5) (layers "F.Cu" "F.Mask" "F.Paste") (solder_mask_margin 0.102))
  (pad "215" smd rect (at -3.825 -2.05 270) (size 0.52 1.5) (layers "F.Cu" "F.Mask" "F.Paste") (solder_mask_margin 0.102))
  (pad "216" smd rect (at -2.975 -2.05 270) (size 0.52 1.5) (layers "F.Cu" "F.Mask" "F.Paste") (solder_mask_margin 0.102))
  (pad "217" smd rect (at -2.125 -2.05 270) (size 0.52 1.5) (layers "F.Cu" "F.Mask" "F.Paste") (solder_mask_margin 0.102))
  (pad "218" smd rect (at -1.275 -2.05 270) (size 0.52 1.5) (layers "F.Cu" "F.Mask" "F.Paste") (solder_mask_margin 0.102))
  (pad "219" smd rect (at -0.425 -2.05 270) (size 0.52 1.5) (layers "F.Cu" "F.Mask" "F.Paste") (solder_mask_margin 0.102))
  (pad "220" smd rect (at 5.525 -2.05 270) (size 0.52 1.5) (layers "F.Cu" "F.Mask" "F.Paste") (solder_mask_margin 0.102))
  (pad "221" smd rect (at 6.375 -2.05 270) (size 0.52 1.5) (layers "F.Cu" "F.Mask" "F.Paste") (solder_mask_margin 0.102))
  (pad "222" smd rect (at 7.225 -2.05 270) (size 0.52 1.5) (layers "F.Cu" "F.Mask" "F.Paste") (solder_mask_margin 0.102))
  (pad "223" smd rect (at 8.075 -2.05 270) (size 0.52 1.5) (layers "F.Cu" "F.Mask" "F.Paste") (solder_mask_margin 0.102))
  (pad "224" smd rect (at 8.925 -2.05 270) (size 0.52 1.5) (layers "F.Cu" "F.Mask" "F.Paste") (solder_mask_margin 0.102))
  (pad "225" smd rect (at 9.775 -2.05 270) (size 0.52 1.5) (layers "F.Cu" "F.Mask" "F.Paste") (solder_mask_margin 0.102))
  (pad "226" smd rect (at 10.625 -2.05 270) (size 0.52 1.5) (layers "F.Cu" "F.Mask" "F.Paste") (solder_mask_margin 0.102))
  (pad "227" smd rect (at 11.475 -2.05 270) (size 0.52 1.5) (layers "F.Cu" "F.Mask" "F.Paste") (solder_mask_margin 0.102))
  (pad "228" smd rect (at 12.325 -2.05 270) (size 0.52 1.5) (layers "F.Cu" "F.Mask" "F.Paste") (solder_mask_margin 0.102))
  (pad "229" smd rect (at 13.175 -2.05 270) (size 0.52 1.5) (layers "F.Cu" "F.Mask" "F.Paste") (solder_mask_margin 0.102))
  (pad "230" smd rect (at 14.025 -2.05 270) (size 0.52 1.5) (layers "F.Cu" "F.Mask" "F.Paste") (solder_mask_margin 0.102))
  (pad "231" smd rect (at 14.875 -2.05 270) (size 0.52 1.5) (layers "F.Cu" "F.Mask" "F.Paste") (solder_mask_margin 0.102))
  (pad "232" smd rect (at 15.725 -2.05 270) (size 0.52 1.5) (layers "F.Cu" "F.Mask" "F.Paste") (solder_mask_margin 0.102))
  (pad "233" smd rect (at 16.575 -2.05 270) (size 0.52 1.5) (layers "F.Cu" "F.Mask" "F.Paste") (solder_mask_margin 0.102))
  (pad "234" smd rect (at 17.425 -2.05 270) (size 0.52 1.5) (layers "F.Cu" "F.Mask" "F.Paste") (solder_mask_margin 0.102))
  (pad "235" smd rect (at 18.275 -2.05 270) (size 0.52 1.5) (layers "F.Cu" "F.Mask" "F.Paste") (solder_mask_margin 0.102))
  (pad "236" smd rect (at 19.125 -2.05 270) (size 0.52 1.5) (layers "F.Cu" "F.Mask" "F.Paste") (solder_mask_margin 0.102))
  (pad "237" smd rect (at 19.975 -2.05 270) (size 0.52 1.5) (layers "F.Cu" "F.Mask" "F.Paste") (solder_mask_margin 0.102))
  (pad "238" smd rect (at 20.825 -2.05 270) (size 0.52 1.5) (layers "F.Cu" "F.Mask" "F.Paste") (solder_mask_margin 0.102))
  (pad "239" smd rect (at 21.675 -2.05 270) (size 0.52 1.5) (layers "F.Cu" "F.Mask" "F.Paste") (solder_mask_margin 0.102))
  (pad "240" smd rect (at 22.525 -2.05 270) (size 0.52 1.5) (layers "F.Cu" "F.Mask" "F.Paste") (solder_mask_margin 0.102))
  (pad "241" smd rect (at 23.375 -2.05 270) (size 0.52 1.5) (layers "F.Cu" "F.Mask" "F.Paste") (solder_mask_margin 0.102))
  (pad "242" smd rect (at 24.225 -2.05 270) (size 0.52 1.5) (layers "F.Cu" "F.Mask" "F.Paste") (solder_mask_margin 0.102))
  (pad "243" smd rect (at 25.075 -2.05 270) (size 0.52 1.5) (layers "F.Cu" "F.Mask" "F.Paste") (solder_mask_margin 0.102))
  (pad "244" smd rect (at 25.925 -2.05 270) (size 0.52 1.5) (layers "F.Cu" "F.Mask" "F.Paste") (solder_mask_margin 0.102))
  (pad "245" smd rect (at 26.775 -2.05 270) (size 0.52 1.5) (layers "F.Cu" "F.Mask" "F.Paste") (solder_mask_margin 0.102))
  (pad "246" smd rect (at 27.625 -2.05 270) (size 0.52 1.5) (layers "F.Cu" "F.Mask" "F.Paste") (solder_mask_margin 0.102))
  (pad "247" smd rect (at 28.475 -2.05 270) (size 0.52 1.5) (layers "F.Cu" "F.Mask" "F.Paste") (solder_mask_margin 0.102))
  (pad "248" smd rect (at 29.325 -2.05 270) (size 0.52 1.5) (layers "F.Cu" "F.Mask" "F.Paste") (solder_mask_margin 0.102))
  (pad "249" smd rect (at 30.175 -2.05 270) (size 0.52 1.5) (layers "F.Cu" "F.Mask" "F.Paste") (solder_mask_margin 0.102))
  (pad "250" smd rect (at 31.025 -2.05 270) (size 0.52 1.5) (layers "F.Cu" "F.Mask" "F.Paste") (solder_mask_margin 0.102))
  (pad "251" smd rect (at 31.875 -2.05 270) (size 0.52 1.5) (layers "F.Cu" "F.Mask" "F.Paste") (solder_mask_margin 0.102))
  (pad "252" smd rect (at 32.725 -2.05 270) (size 0.52 1.5) (layers "F.Cu" "F.Mask" "F.Paste") (solder_mask_margin 0.102))
  (pad "253" smd rect (at 33.575 -2.05 270) (size 0.52 1.5) (layers "F.Cu" "F.Mask" "F.Paste") (solder_mask_margin 0.102))
  (pad "254" smd rect (at 34.425 -2.05 270) (size 0.52 1.5) (layers "F.Cu" "F.Mask" "F.Paste") (solder_mask_margin 0.102))
  (pad "255" smd rect (at 35.275 -2.05 270) (size 0.52 1.5) (layers "F.Cu" "F.Mask" "F.Paste") (solder_mask_margin 0.102))
  (pad "256" smd rect (at 36.125 -2.05 270) (size 0.52 1.5) (layers "F.Cu" "F.Mask" "F.Paste") (solder_mask_margin 0.102))
  (pad "257" smd rect (at 36.975 -2.05 270) (size 0.52 1.5) (layers "F.Cu" "F.Mask" "F.Paste") (solder_mask_margin 0.102))
  (pad "258" smd rect (at 37.825 -2.05 270) (size 0.52 1.5) (layers "F.Cu" "F.Mask" "F.Paste") (solder_mask_margin 0.102))
  (pad "259" smd rect (at 38.675 -2.05 270) (size 0.52 1.5) (layers "F.Cu" "F.Mask" "F.Paste") (solder_mask_margin 0.102))
  (pad "260" smd rect (at 39.525 -2.05 270) (size 0.52 1.5) (layers "F.Cu" "F.Mask" "F.Paste") (solder_mask_margin 0.102))
  (pad "261" smd rect (at 40.375 -2.05 270) (size 0.52 1.5) (layers "F.Cu" "F.Mask" "F.Paste") (solder_mask_margin 0.102))
  (pad "262" smd rect (at 41.225 -2.05 270) (size 0.52 1.5) (layers "F.Cu" "F.Mask" "F.Paste") (solder_mask_margin 0.102))
  (pad "263" smd rect (at 42.075 -2.05 270) (size 0.52 1.5) (layers "F.Cu" "F.Mask" "F.Paste") (solder_mask_margin 0.102))
  (pad "264" smd rect (at 42.925 -2.05 270) (size 0.52 1.5) (layers "F.Cu" "F.Mask" "F.Paste") (solder_mask_margin 0.102))
  (pad "265" smd rect (at 43.775 -2.05 270) (size 0.52 1.5) (layers "F.Cu" "F.Mask" "F.Paste") (solder_mask_margin 0.102))
  (pad "266" smd rect (at 44.625 -2.05 270) (size 0.52 1.5) (layers "F.Cu" "F.Mask" "F.Paste") (solder_mask_margin 0.102))
  (pad "267" smd rect (at 45.475 -2.05 270) (size 0.52 1.5) (layers "F.Cu" "F.Mask" "F.Paste") (solder_mask_margin 0.102))
  (pad "268" smd rect (at 46.325 -2.05 270) (size 0.52 1.5) (layers "F.Cu" "F.Mask" "F.Paste") (solder_mask_margin 0.102))
  (pad "269" smd rect (at 47.175 -2.05 270) (size 0.52 1.5) (layers "F.Cu" "F.Mask" "F.Paste") (solder_mask_margin 0.102))
  (pad "270" smd rect (at 48.025 -2.05 270) (size 0.52 1.5) (layers "F.Cu" "F.Mask" "F.Paste") (solder_mask_margin 0.102))
  (pad "271" smd rect (at 48.875 -2.05 270) (size 0.52 1.5) (layers "F.Cu" "F.Mask" "F.Paste") (solder_mask_margin 0.102))
  (pad "272" smd rect (at 49.725 -2.05 270) (size 0.52 1.5) (layers "F.Cu" "F.Mask" "F.Paste") (solder_mask_margin 0.102))
  (pad "273" smd rect (at 50.575 -2.05 270) (size 0.52 1.5) (layers "F.Cu" "F.Mask" "F.Paste") (solder_mask_margin 0.102))
  (pad "274" smd rect (at 51.425 -2.05 270) (size 0.52 1.5) (layers "F.Cu" "F.Mask" "F.Paste") (solder_mask_margin 0.102))
  (pad "275" smd rect (at 52.275 -2.05 270) (size 0.52 1.5) (layers "F.Cu" "F.Mask" "F.Paste") (solder_mask_margin 0.102))
  (pad "276" smd rect (at 53.125 -2.05 270) (size 0.52 1.5) (layers "F.Cu" "F.Mask" "F.Paste") (solder_mask_margin 0.102))
  (pad "277" smd rect (at 53.975 -2.05 270) (size 0.52 1.5) (layers "F.Cu" "F.Mask" "F.Paste") (solder_mask_margin 0.102))
  (pad "278" smd rect (at 54.825 -2.05 270) (size 0.52 1.5) (layers "F.Cu" "F.Mask" "F.Paste") (solder_mask_margin 0.102))
  (pad "279" smd rect (at 55.675 -2.05 270) (size 0.52 1.5) (layers "F.Cu" "F.Mask" "F.Paste") (solder_mask_margin 0.102))
  (pad "280" smd rect (at 56.525 -2.05 270) (size 0.52 1.5) (layers "F.Cu" "F.Mask" "F.Paste") (solder_mask_margin 0.102))
  (pad "281" smd rect (at 57.375 -2.05 270) (size 0.52 1.5) (layers "F.Cu" "F.Mask" "F.Paste") (solder_mask_margin 0.102))
  (pad "282" smd rect (at 58.225 -2.05 270) (size 0.52 1.5) (layers "F.Cu" "F.Mask" "F.Paste") (solder_mask_margin 0.102))
  (pad "283" smd rect (at 59.075 -2.05 270) (size 0.52 1.5) (layers "F.Cu" "F.Mask" "F.Paste") (solder_mask_margin 0.102))
  (pad "284" smd rect (at 59.925 -2.05 270) (size 0.52 1.5) (layers "F.Cu" "F.Mask" "F.Paste") (solder_mask_margin 0.102))
  (pad "285" smd rect (at 60.775 -2.05 270) (size 0.52 1.5) (layers "F.Cu" "F.Mask" "F.Paste") (solder_mask_margin 0.102))
  (pad "286" smd rect (at 61.625 -2.05 270) (size 0.52 1.5) (layers "F.Cu" "F.Mask" "F.Paste") (solder_mask_margin 0.102))
  (pad "287" smd rect (at 62.475 -2.05 270) (size 0.52 1.5) (layers "F.Cu" "F.Mask" "F.Paste") (solder_mask_margin 0.102))
  (pad "288" smd rect (at 63.325 -2.05 270) (size 0.52 1.5) (layers "F.Cu" "F.Mask" "F.Paste") (solder_mask_margin 0.102))
  (pad "S1" thru_hole oval (at -68.975 0 270) (size 1.875 3.75) (drill oval 1.25 2.53) (layers "*.Cu" "*.Mask") (remove_unused_layers no)
   (solder_mask_margin 0.102))
  (pad "S2" thru_hole oval (at 1.425 0 270) (size 1.875 3.75) (drill oval 1.25 2.53) (layers "*.Cu" "*.Mask") (remove_unused_layers no)
   (solder_mask_margin 0.102))
  (pad "S3" thru_hole oval (at 68.975 0 270) (size 1.875 3.75) (drill oval 1.25 2.53) (layers "*.Cu" "*.Mask") (remove_unused_layers no)
   (solder_mask_margin 0.102)))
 (gr_line (start 2.5 2.5) (end 17.18425 2.5) (stroke (width 0.1) (type default)) (layer "Edge.Cuts"))
 (gr_line (start 2.5 166.05) (end 2.5 2.5) (stroke (width 0.1) (type default)) (layer "Edge.Cuts"))
 (gr_line (start 17.18425 2.5) (end 17.18425 166.05) (stroke (width 0.1) (type default)) (layer "Edge.Cuts"))
 (gr_line (start 17.18425 166.05) (end 2.5 166.05) (stroke (width 0.1) (type default)) (layer "Edge.Cuts"))
 (segment (start 6.851 20.95) (end 10.951 20.95) (width 0.8128) (layer "F.Cu") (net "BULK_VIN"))
 (segment (start 10.951 21.8) (end 10.951 20.95) (width 0.8128) (layer "F.Cu") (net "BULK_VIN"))
 (segment (start 13.151 71.475) (end 13.151 72.525) (width 0.6096) (layer "F.Cu") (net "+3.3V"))
 (segment (start 13.151 55.275) (end 13.151 71.475) (width 0.6096) (layer "F.Cu") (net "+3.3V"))
 (segment (start 13.151 26.025) (end 13.151 55.275) (width 0.6096) (layer "F.Cu") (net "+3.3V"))
 (segment (start 13.126 26.05) (end 10.951 26.05) (width 0.6096) (layer "F.Cu") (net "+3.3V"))
 (via (at 13.151 71.475) (size 0.6548) (drill 0.35) (layers "F.Cu" "B.Cu") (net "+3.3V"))
 (via (at 13.151 72.525) (size 0.6548) (drill 0.35) (layers "F.Cu" "B.Cu") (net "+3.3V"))
 (segment (start 13.151 72.525) (end 13.151 71.475) (width 0.6096) (layer "B.Cu") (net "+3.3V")))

